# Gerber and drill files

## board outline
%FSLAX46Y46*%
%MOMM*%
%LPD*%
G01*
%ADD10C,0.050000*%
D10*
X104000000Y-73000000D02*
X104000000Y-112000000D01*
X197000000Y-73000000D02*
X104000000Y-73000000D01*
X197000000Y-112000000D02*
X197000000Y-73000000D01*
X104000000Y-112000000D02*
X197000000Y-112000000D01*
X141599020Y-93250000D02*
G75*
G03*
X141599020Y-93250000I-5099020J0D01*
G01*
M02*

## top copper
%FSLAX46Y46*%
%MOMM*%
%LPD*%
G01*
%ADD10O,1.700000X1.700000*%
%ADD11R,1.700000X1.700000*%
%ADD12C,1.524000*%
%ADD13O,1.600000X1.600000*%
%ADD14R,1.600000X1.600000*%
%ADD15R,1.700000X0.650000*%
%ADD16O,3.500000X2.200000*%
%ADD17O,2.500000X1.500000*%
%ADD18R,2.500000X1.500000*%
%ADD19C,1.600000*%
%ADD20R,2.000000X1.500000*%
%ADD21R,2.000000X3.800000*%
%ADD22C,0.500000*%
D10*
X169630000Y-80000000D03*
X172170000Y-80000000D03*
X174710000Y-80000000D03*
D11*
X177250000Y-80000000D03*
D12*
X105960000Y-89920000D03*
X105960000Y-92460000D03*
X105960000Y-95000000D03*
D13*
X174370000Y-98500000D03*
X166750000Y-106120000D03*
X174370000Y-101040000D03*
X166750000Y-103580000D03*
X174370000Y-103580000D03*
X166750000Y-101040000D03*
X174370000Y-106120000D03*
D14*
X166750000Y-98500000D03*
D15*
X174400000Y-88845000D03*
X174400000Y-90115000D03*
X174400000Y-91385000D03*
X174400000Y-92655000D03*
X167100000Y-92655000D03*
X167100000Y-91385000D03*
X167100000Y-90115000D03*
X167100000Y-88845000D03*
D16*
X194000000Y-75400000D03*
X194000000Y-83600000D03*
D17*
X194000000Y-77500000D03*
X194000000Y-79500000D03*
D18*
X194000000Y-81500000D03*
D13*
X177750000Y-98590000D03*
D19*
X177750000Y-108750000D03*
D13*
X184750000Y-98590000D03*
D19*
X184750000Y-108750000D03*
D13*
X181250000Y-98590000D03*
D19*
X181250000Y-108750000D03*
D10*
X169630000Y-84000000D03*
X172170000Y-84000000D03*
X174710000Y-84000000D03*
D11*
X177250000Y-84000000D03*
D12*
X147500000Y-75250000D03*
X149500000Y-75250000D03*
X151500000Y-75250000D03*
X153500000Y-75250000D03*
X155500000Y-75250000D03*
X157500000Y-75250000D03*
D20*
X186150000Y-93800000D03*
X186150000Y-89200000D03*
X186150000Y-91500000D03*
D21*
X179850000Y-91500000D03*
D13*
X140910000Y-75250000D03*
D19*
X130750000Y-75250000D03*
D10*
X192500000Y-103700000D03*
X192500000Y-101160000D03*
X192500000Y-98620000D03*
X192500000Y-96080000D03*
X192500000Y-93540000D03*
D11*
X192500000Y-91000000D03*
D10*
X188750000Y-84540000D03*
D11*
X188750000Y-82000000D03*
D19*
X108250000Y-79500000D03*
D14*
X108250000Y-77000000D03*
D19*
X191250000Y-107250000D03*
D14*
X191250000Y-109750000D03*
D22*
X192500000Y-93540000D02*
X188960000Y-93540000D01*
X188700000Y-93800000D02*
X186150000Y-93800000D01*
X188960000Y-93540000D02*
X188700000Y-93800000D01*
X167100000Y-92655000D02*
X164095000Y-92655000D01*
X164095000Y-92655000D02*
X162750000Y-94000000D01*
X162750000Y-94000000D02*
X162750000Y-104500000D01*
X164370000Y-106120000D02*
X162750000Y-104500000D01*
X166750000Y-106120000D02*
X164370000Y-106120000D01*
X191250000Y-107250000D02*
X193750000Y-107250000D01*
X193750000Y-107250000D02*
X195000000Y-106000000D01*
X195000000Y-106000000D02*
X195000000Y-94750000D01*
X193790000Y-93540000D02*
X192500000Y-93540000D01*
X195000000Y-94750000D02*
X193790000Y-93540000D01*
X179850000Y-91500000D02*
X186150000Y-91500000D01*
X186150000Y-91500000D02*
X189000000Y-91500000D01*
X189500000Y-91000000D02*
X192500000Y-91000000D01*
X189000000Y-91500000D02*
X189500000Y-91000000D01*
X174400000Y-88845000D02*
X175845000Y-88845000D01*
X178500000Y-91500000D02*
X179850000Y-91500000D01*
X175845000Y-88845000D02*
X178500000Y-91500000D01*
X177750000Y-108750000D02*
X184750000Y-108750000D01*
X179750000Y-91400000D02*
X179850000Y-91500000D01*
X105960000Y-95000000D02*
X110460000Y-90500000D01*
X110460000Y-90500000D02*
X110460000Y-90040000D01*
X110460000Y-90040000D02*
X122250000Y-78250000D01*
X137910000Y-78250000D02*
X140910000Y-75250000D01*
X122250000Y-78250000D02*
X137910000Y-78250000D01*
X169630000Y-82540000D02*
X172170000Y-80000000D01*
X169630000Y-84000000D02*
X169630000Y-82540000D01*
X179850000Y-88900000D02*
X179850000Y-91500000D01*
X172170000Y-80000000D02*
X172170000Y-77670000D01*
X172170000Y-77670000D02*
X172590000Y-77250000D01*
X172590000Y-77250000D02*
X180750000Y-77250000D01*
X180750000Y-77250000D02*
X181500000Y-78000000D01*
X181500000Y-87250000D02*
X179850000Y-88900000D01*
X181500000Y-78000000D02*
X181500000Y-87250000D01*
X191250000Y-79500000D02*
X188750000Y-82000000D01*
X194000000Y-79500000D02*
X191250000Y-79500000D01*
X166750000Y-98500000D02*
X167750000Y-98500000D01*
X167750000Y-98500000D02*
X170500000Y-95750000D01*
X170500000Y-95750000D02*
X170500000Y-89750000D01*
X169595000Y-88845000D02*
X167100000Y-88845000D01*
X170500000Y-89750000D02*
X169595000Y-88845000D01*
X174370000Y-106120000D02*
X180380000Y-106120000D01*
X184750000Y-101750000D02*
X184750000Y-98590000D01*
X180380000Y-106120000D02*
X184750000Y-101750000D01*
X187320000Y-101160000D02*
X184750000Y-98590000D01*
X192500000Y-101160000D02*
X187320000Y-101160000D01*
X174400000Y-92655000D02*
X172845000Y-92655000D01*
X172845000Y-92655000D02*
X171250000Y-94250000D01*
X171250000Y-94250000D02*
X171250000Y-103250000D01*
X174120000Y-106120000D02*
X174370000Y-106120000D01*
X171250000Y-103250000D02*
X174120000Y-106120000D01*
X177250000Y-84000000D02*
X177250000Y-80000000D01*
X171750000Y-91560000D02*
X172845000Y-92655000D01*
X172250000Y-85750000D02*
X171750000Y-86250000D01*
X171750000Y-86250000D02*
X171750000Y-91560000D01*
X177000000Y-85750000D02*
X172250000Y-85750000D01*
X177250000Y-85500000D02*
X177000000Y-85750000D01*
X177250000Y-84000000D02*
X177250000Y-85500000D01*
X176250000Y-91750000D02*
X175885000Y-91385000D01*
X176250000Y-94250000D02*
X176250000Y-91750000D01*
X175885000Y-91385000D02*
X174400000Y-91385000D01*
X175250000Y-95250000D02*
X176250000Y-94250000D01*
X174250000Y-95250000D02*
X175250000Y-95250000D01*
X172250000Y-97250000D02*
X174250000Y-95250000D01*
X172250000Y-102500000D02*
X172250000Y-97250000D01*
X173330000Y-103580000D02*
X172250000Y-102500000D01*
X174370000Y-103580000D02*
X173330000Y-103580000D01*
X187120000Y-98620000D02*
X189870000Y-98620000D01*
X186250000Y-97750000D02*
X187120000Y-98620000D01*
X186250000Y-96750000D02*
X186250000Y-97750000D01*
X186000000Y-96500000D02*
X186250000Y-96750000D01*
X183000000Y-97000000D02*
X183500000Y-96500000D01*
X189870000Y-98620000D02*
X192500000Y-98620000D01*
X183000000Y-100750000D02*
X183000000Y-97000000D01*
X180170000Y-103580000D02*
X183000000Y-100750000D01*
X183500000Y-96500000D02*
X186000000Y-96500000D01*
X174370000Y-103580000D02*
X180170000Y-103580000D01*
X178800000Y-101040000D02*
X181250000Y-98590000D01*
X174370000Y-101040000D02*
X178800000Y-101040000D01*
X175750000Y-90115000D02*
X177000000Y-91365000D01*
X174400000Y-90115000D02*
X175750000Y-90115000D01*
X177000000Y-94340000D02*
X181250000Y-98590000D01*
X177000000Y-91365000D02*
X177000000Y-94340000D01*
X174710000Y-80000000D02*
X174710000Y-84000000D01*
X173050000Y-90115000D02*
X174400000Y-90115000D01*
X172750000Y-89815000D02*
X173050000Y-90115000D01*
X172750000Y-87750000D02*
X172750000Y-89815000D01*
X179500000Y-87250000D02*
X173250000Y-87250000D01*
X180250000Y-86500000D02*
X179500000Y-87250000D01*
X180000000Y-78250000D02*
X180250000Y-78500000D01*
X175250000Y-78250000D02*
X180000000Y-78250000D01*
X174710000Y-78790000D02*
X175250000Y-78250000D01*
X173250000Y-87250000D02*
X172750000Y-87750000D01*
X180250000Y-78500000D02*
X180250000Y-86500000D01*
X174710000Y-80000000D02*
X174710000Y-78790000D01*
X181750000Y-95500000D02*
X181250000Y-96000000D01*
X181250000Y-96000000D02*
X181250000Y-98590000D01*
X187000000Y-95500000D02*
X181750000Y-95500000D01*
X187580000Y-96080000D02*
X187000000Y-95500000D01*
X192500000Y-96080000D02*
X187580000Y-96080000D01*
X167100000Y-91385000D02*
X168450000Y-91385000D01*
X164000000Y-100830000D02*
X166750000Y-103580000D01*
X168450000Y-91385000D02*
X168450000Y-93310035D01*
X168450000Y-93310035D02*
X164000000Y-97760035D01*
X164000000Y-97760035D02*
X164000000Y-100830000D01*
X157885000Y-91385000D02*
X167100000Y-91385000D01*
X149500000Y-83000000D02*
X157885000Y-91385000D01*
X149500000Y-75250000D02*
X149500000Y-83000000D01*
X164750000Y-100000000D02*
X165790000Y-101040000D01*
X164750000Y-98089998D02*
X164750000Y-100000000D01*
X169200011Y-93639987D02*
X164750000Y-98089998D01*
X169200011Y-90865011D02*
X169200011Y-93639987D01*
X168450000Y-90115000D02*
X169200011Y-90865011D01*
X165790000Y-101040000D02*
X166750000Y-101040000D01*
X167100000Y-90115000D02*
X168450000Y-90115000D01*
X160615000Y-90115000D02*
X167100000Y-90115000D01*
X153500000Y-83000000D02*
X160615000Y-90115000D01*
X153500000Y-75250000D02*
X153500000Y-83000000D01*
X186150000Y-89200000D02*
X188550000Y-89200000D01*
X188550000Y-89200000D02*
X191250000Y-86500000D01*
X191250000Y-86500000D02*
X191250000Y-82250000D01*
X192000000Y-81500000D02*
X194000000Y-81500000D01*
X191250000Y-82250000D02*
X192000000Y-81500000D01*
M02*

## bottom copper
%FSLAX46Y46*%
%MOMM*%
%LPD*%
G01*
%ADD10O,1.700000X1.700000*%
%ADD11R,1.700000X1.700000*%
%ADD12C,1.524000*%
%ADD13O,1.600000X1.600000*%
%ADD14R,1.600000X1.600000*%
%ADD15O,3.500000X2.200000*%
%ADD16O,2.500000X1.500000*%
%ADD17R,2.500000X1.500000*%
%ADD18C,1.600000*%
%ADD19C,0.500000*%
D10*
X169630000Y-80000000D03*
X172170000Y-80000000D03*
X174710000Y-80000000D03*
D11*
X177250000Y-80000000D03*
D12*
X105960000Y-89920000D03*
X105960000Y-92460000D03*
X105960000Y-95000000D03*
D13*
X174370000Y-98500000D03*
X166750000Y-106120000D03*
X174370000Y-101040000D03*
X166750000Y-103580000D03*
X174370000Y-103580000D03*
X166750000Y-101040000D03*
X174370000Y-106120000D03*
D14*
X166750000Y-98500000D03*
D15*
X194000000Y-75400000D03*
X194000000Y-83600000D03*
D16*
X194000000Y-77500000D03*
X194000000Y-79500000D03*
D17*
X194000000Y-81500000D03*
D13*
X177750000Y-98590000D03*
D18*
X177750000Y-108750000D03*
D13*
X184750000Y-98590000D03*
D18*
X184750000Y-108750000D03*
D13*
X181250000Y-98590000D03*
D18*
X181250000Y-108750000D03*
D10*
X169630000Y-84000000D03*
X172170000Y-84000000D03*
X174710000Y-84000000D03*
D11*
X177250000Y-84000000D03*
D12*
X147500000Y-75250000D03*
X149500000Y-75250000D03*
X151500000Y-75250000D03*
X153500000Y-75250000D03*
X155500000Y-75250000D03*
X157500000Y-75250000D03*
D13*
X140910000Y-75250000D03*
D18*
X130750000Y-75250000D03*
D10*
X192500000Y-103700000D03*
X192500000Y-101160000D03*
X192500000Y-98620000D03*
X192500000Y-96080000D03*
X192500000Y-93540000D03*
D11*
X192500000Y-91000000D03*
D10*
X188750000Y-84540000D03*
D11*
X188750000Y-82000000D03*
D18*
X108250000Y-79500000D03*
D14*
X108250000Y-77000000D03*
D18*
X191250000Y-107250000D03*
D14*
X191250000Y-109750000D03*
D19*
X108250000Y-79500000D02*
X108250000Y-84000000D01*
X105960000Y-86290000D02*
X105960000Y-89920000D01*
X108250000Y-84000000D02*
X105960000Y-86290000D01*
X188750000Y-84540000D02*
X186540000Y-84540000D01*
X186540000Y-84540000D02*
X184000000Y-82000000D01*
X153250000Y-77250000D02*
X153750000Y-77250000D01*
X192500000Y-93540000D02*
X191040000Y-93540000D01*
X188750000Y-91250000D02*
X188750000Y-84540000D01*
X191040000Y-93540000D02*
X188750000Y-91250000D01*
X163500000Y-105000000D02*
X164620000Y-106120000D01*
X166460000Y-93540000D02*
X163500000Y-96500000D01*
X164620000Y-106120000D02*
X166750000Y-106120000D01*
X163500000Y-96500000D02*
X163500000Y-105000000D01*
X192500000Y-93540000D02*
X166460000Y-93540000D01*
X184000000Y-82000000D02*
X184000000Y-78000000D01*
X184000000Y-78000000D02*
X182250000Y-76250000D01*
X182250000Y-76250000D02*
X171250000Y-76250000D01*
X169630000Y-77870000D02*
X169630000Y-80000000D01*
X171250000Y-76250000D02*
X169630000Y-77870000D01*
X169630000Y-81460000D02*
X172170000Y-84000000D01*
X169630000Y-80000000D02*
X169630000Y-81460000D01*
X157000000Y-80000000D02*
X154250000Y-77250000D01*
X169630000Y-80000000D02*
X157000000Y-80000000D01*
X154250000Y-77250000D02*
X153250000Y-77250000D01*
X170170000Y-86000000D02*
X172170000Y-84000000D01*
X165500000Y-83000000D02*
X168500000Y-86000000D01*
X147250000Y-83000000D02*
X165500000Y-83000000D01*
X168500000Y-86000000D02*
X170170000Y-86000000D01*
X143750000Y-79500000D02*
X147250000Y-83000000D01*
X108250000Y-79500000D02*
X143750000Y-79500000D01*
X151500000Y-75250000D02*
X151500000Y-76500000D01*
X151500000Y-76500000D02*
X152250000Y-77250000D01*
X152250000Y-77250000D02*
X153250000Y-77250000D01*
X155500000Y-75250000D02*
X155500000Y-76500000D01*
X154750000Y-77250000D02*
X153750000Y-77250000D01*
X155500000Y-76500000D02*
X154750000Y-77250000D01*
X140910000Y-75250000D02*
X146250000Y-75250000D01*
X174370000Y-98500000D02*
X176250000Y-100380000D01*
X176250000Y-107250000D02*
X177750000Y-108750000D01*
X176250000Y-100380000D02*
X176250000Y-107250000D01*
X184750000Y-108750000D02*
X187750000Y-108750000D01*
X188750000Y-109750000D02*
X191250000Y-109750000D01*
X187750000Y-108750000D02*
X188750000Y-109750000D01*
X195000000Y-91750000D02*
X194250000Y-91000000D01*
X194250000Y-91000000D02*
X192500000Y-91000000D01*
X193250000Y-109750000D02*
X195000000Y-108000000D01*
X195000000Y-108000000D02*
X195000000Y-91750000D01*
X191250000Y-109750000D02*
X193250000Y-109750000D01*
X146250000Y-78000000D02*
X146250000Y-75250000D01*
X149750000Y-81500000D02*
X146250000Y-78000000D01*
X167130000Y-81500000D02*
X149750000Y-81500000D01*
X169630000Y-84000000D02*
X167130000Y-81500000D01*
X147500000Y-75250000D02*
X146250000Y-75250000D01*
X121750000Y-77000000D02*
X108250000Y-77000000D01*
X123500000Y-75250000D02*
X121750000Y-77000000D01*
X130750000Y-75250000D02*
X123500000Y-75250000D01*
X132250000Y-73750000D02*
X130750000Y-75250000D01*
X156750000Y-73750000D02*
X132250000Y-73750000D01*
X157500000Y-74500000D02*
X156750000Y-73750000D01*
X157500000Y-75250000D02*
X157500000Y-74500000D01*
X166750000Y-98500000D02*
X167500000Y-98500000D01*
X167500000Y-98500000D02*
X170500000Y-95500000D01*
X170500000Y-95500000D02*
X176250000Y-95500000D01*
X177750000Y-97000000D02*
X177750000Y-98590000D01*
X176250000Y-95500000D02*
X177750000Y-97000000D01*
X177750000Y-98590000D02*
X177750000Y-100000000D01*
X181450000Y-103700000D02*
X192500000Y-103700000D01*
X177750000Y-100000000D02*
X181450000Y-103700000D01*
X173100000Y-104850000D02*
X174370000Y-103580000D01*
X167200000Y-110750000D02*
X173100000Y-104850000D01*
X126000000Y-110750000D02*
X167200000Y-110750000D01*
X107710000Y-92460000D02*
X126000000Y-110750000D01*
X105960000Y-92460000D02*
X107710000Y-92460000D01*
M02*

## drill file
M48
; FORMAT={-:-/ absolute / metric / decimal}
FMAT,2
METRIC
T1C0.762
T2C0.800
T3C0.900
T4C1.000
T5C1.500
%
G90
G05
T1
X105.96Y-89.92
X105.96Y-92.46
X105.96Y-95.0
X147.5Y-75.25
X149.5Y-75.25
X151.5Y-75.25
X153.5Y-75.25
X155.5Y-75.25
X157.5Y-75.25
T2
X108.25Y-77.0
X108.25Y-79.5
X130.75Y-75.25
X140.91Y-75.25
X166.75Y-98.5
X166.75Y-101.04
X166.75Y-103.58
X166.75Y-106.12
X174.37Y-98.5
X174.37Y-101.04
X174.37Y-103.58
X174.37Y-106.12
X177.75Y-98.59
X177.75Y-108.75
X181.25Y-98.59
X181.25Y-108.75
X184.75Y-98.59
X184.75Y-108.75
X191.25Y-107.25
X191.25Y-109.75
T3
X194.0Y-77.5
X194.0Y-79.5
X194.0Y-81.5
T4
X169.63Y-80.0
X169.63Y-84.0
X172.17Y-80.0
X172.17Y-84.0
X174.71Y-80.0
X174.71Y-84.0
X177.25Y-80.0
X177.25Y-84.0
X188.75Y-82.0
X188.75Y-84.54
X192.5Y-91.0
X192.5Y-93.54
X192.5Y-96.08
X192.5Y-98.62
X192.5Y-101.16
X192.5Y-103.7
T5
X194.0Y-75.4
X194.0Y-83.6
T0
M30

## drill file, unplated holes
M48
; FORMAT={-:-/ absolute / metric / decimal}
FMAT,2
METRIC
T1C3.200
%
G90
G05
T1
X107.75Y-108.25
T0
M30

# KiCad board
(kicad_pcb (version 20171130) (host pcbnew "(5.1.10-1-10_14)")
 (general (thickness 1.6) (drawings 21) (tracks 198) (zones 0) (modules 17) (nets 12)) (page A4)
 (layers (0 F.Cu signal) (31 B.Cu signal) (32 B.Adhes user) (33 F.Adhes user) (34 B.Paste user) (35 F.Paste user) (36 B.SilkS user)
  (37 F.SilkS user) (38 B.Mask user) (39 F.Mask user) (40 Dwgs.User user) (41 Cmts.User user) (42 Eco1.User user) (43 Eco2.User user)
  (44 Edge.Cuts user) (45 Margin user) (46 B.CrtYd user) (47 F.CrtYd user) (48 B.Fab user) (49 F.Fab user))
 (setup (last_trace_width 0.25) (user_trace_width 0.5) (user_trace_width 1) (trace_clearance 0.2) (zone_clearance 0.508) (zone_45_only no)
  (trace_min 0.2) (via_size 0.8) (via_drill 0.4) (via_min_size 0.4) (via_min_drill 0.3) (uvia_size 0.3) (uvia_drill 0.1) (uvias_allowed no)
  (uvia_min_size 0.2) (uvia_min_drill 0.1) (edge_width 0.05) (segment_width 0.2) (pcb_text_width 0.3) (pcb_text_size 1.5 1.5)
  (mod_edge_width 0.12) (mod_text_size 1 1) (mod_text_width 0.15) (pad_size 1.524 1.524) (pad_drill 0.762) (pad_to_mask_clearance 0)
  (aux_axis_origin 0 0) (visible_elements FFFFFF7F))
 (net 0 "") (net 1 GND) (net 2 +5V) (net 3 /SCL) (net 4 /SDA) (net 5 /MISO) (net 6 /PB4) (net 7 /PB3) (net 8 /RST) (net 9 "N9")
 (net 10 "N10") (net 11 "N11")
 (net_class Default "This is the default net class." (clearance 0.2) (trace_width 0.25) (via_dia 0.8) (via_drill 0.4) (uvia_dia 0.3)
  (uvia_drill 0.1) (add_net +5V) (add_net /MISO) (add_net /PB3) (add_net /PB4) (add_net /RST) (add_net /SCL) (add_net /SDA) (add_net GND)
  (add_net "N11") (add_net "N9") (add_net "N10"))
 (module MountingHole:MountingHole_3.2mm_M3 (layer F.Cu) (at 107.75 108.25)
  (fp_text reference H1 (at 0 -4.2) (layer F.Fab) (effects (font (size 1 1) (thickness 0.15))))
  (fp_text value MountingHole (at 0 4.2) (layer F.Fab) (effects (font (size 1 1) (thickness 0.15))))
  (pad 1 np_thru_hole circle (at 0 0) (size 3.2 3.2) (drill 3.2) (layers *.Cu *.Mask)))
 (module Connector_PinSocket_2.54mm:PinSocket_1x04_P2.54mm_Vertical (layer F.Cu) (at 177.25 80 270)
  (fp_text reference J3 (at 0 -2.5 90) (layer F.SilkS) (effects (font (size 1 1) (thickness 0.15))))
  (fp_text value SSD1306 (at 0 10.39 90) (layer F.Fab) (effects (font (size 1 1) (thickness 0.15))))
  (pad 4 thru_hole oval (at 0 7.62 270) (size 1.7 1.7) (drill 1) (layers *.Cu *.Mask) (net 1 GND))
  (pad 3 thru_hole oval (at 0 5.08 270) (size 1.7 1.7) (drill 1) (layers *.Cu *.Mask) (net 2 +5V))
  (pad 2 thru_hole oval (at 0 2.54 270) (size 1.7 1.7) (drill 1) (layers *.Cu *.Mask) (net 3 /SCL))
  (pad 1 thru_hole rect (at 0 0 270) (size 1.7 1.7) (drill 1) (layers *.Cu *.Mask) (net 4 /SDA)))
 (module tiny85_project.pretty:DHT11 (layer F.Cu) (at 104.5 86 270)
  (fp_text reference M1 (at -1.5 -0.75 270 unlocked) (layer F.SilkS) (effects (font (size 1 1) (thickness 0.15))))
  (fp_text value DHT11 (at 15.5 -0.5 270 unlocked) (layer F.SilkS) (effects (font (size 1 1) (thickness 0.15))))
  (pad 3 thru_hole circle (at 3.92 -1.46 90) (size 1.524 1.524) (drill 0.762) (layers *.Cu *.Mask) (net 1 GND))
  (pad 2 thru_hole circle (at 6.46 -1.46 90) (size 1.524 1.524) (drill 0.762) (layers *.Cu *.Mask) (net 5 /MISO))
  (pad 1 thru_hole circle (at 9 -1.46 90) (size 1.524 1.524) (drill 0.762) (layers *.Cu *.Mask) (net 2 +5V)))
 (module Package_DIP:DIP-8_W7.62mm (layer F.Cu) (at 166.75 98.5)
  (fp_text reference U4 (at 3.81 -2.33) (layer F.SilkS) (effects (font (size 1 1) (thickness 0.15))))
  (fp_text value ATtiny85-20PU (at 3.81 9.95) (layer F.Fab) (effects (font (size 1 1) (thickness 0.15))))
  (pad 8 thru_hole oval (at 7.62 0) (size 1.6 1.6) (drill 0.8) (layers *.Cu *.Mask) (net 2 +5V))
  (pad 4 thru_hole oval (at 0 7.62) (size 1.6 1.6) (drill 0.8) (layers *.Cu *.Mask) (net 1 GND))
  (pad 7 thru_hole oval (at 7.62 2.54) (size 1.6 1.6) (drill 0.8) (layers *.Cu *.Mask) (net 3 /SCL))
  (pad 3 thru_hole oval (at 0 5.08) (size 1.6 1.6) (drill 0.8) (layers *.Cu *.Mask) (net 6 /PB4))
  (pad 6 thru_hole oval (at 7.62 5.08) (size 1.6 1.6) (drill 0.8) (layers *.Cu *.Mask) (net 5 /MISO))
  (pad 2 thru_hole oval (at 0 2.54) (size 1.6 1.6) (drill 0.8) (layers *.Cu *.Mask) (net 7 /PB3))
  (pad 5 thru_hole oval (at 7.62 7.62) (size 1.6 1.6) (drill 0.8) (layers *.Cu *.Mask) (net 4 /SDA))
  (pad 1 thru_hole rect (at 0 0) (size 1.6 1.6) (drill 0.8) (layers *.Cu *.Mask) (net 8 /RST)))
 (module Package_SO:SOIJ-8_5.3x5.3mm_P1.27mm (layer F.Cu) (at 170.75 90.75)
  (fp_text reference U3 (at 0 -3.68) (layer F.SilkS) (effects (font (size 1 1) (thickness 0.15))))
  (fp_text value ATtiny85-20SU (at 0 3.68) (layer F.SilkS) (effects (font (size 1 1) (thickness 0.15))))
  (pad 8 smd rect (at 3.65 -1.905) (size 1.7 0.65) (layers F.Cu F.Paste F.Mask) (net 2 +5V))
  (pad 7 smd rect (at 3.65 -0.635) (size 1.7 0.65) (layers F.Cu F.Paste F.Mask) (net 3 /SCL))
  (pad 6 smd rect (at 3.65 0.635) (size 1.7 0.65) (layers F.Cu F.Paste F.Mask) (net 5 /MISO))
  (pad 5 smd rect (at 3.65 1.905) (size 1.7 0.65) (layers F.Cu F.Paste F.Mask) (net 4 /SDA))
  (pad 4 smd rect (at -3.65 1.905) (size 1.7 0.65) (layers F.Cu F.Paste F.Mask) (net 1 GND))
  (pad 3 smd rect (at -3.65 0.635) (size 1.7 0.65) (layers F.Cu F.Paste F.Mask) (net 6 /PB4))
  (pad 2 smd rect (at -3.65 -0.635) (size 1.7 0.65) (layers F.Cu F.Paste F.Mask) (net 7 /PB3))
  (pad 1 smd rect (at -3.65 -1.905) (size 1.7 0.65) (layers F.Cu F.Paste F.Mask) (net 8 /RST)))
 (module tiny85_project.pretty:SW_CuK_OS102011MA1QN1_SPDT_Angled (layer F.Cu) (at 194 81.5 90)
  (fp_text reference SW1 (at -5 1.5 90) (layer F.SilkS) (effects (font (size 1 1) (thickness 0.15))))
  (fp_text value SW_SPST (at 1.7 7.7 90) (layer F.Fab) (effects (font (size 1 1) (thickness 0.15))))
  (pad "" thru_hole oval (at 6.1 0 90) (size 2.2 3.5) (drill 1.5) (layers *.Cu *.Mask))
  (pad "" thru_hole oval (at -2.1 0 90) (size 2.2 3.5) (drill 1.5) (layers *.Cu *.Mask))
  (pad 3 thru_hole oval (at 4 0 90) (size 1.5 2.5) (drill 0.9) (layers *.Cu *.Mask))
  (pad 2 thru_hole oval (at 2 0 90) (size 1.5 2.5) (drill 0.9) (layers *.Cu *.Mask) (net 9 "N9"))
  (pad 1 thru_hole rect (at 0 0 90) (size 1.5 2.5) (drill 0.9) (layers *.Cu *.Mask) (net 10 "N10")))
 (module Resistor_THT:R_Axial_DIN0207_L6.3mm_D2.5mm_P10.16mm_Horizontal (layer F.Cu) (at 177.75 108.75 90)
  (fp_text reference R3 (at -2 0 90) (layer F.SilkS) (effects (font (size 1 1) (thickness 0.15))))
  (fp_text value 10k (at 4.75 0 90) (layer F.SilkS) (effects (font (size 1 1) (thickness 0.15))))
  (pad 2 thru_hole oval (at 10.16 0 90) (size 1.6 1.6) (drill 0.8) (layers *.Cu *.Mask) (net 8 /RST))
  (pad 1 thru_hole circle (at 0 0 90) (size 1.6 1.6) (drill 0.8) (layers *.Cu *.Mask) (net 2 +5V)))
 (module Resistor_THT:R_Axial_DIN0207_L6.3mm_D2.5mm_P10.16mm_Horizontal (layer F.Cu) (at 184.75 108.75 90)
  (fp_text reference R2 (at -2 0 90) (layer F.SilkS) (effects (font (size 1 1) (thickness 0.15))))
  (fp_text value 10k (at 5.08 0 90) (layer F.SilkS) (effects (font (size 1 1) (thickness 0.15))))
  (pad 2 thru_hole oval (at 10.16 0 90) (size 1.6 1.6) (drill 0.8) (layers *.Cu *.Mask) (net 4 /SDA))
  (pad 1 thru_hole circle (at 0 0 90) (size 1.6 1.6) (drill 0.8) (layers *.Cu *.Mask) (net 2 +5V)))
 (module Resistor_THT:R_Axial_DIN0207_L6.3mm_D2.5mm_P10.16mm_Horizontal (layer F.Cu) (at 181.25 108.75 90)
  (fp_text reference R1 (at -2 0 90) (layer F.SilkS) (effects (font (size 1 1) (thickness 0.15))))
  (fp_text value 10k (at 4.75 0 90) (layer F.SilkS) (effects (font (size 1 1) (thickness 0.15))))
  (pad 2 thru_hole oval (at 10.16 0 90) (size 1.6 1.6) (drill 0.8) (layers *.Cu *.Mask) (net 3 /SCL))
  (pad 1 thru_hole circle (at 0 0 90) (size 1.6 1.6) (drill 0.8) (layers *.Cu *.Mask) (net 2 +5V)))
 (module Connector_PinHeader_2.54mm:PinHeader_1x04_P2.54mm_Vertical (layer F.Cu) (at 177.25 84 270)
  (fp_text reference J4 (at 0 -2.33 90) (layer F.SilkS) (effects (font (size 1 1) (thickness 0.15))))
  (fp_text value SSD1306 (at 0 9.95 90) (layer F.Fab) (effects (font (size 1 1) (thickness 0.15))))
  (pad 4 thru_hole oval (at 0 7.62 270) (size 1.7 1.7) (drill 1) (layers *.Cu *.Mask) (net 2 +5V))
  (pad 3 thru_hole oval (at 0 5.08 270) (size 1.7 1.7) (drill 1) (layers *.Cu *.Mask) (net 1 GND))
  (pad 2 thru_hole oval (at 0 2.54 270) (size 1.7 1.7) (drill 1) (layers *.Cu *.Mask) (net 3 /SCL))
  (pad 1 thru_hole rect (at 0 0 270) (size 1.7 1.7) (drill 1) (layers *.Cu *.Mask) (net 4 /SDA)))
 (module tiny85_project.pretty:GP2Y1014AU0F (layer F.Cu) (at 159.5 77.25 180)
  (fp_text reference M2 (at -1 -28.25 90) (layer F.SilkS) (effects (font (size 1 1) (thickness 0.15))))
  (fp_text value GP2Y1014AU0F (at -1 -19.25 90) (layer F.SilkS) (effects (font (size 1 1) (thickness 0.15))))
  (pad 6 thru_hole circle (at 12 2 180) (size 1.524 1.524) (drill 0.762) (layers *.Cu *.Mask) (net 2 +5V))
  (pad 5 thru_hole circle (at 10 2 180) (size 1.524 1.524) (drill 0.762) (layers *.Cu *.Mask) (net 6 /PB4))
  (pad 4 thru_hole circle (at 8 2 180) (size 1.524 1.524) (drill 0.762) (layers *.Cu *.Mask) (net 1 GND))
  (pad 3 thru_hole circle (at 6 2 180) (size 1.524 1.524) (drill 0.762) (layers *.Cu *.Mask) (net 7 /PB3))
  (pad 2 thru_hole circle (at 4 2 180) (size 1.524 1.524) (drill 0.762) (layers *.Cu *.Mask) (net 1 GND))
  (pad 1 thru_hole circle (at 2 2 180) (size 1.524 1.524) (drill 0.762) (layers *.Cu *.Mask) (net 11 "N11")))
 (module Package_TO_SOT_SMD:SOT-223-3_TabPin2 (layer F.Cu) (at 183 91.5 180)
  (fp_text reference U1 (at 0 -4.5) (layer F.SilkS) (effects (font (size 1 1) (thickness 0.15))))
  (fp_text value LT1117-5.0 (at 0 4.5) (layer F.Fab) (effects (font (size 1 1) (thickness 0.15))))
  (pad 1 smd rect (at -3.15 -2.3 180) (size 2 1.5) (layers F.Cu F.Paste F.Mask) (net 1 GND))
  (pad 3 smd rect (at -3.15 2.3 180) (size 2 1.5) (layers F.Cu F.Paste F.Mask) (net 10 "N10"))
  (pad 2 smd rect (at -3.15 0 180) (size 2 1.5) (layers F.Cu F.Paste F.Mask) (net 2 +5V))
  (pad 2 smd rect (at 3.15 0 180) (size 2 3.8) (layers F.Cu F.Paste F.Mask) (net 2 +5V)))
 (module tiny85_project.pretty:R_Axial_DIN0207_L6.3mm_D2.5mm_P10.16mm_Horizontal (layer F.Cu) (at 130.75 75.25)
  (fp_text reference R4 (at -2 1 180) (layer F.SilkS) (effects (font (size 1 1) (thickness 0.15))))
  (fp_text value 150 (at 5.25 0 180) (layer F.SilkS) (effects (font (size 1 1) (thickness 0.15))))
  (pad 2 thru_hole oval (at 10.16 0) (size 1.6 1.6) (drill 0.8) (layers *.Cu *.Mask) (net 2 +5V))
  (pad 1 thru_hole circle (at 0 0) (size 1.6 1.6) (drill 0.8) (layers *.Cu *.Mask) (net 11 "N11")))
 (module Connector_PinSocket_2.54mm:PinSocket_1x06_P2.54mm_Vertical (layer F.Cu) (at 192.5 91)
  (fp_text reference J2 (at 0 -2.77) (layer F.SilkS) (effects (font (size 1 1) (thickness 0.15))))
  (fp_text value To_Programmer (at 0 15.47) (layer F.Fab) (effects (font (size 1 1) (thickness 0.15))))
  (pad 6 thru_hole oval (at 0 12.7) (size 1.7 1.7) (drill 1) (layers *.Cu *.Mask) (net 8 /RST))
  (pad 5 thru_hole oval (at 0 10.16) (size 1.7 1.7) (drill 1) (layers *.Cu *.Mask) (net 4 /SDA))
  (pad 4 thru_hole oval (at 0 7.62) (size 1.7 1.7) (drill 1) (layers *.Cu *.Mask) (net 5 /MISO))
  (pad 3 thru_hole oval (at 0 5.08) (size 1.7 1.7) (drill 1) (layers *.Cu *.Mask) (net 3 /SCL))
  (pad 2 thru_hole oval (at 0 2.54) (size 1.7 1.7) (drill 1) (layers *.Cu *.Mask) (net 1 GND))
  (pad 1 thru_hole rect (at 0 0) (size 1.7 1.7) (drill 1) (layers *.Cu *.Mask) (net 2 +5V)))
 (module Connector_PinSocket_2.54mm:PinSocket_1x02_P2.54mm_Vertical (layer F.Cu) (at 188.75 82)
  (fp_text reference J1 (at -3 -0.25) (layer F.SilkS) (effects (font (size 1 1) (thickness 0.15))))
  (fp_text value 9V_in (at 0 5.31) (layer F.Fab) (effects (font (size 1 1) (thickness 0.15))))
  (pad 2 thru_hole oval (at 0 2.54) (size 1.7 1.7) (drill 1) (layers *.Cu *.Mask) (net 1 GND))
  (pad 1 thru_hole rect (at 0 0) (size 1.7 1.7) (drill 1) (layers *.Cu *.Mask) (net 9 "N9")))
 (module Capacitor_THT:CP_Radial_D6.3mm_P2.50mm (layer F.Cu) (at 108.25 77 270)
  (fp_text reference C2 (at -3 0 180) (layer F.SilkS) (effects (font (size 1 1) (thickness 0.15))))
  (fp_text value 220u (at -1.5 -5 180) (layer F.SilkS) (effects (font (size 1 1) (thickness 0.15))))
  (pad 2 thru_hole circle (at 2.5 0 270) (size 1.6 1.6) (drill 0.8) (layers *.Cu *.Mask) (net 1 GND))
  (pad 1 thru_hole rect (at 0 0 270) (size 1.6 1.6) (drill 0.8) (layers *.Cu *.Mask) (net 11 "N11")))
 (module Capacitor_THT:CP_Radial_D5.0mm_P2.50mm (layer F.Cu) (at 191.25 109.75 90)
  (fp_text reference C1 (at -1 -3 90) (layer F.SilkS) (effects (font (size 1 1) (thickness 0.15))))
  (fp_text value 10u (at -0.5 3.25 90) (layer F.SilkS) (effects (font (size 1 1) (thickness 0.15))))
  (pad 2 thru_hole circle (at 2.5 0 90) (size 1.6 1.6) (drill 0.8) (layers *.Cu *.Mask) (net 1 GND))
  (pad 1 thru_hole rect (at 0 0 90) (size 1.6 1.6) (drill 0.8) (layers *.Cu *.Mask) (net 2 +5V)))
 (gr_line (start 104 73) (end 104 112) (layer Edge.Cuts) (width 0.05))
 (gr_line (start 197 73) (end 104 73) (layer Edge.Cuts) (width 0.05))
 (gr_line (start 197 112) (end 197 73) (layer Edge.Cuts) (width 0.05))
 (gr_line (start 104 112) (end 197 112) (layer Edge.Cuts) (width 0.05))
 (gr_circle (center 136.5 93.25) (end 141.5 94.25) (layer Edge.Cuts) (width 0.05))
 (segment (start 108.25 79.5) (end 108.25 84) (width 0.5) (layer B.Cu) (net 1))
 (segment (start 105.96 86.29) (end 105.96 89.92) (width 0.5) (layer B.Cu) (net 1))
 (segment (start 108.25 84) (end 105.96 86.29) (width 0.5) (layer B.Cu) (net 1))
 (segment (start 192.5 93.54) (end 188.96 93.54) (width 0.5) (layer F.Cu) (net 1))
 (segment (start 188.7 93.8) (end 186.15 93.8) (width 0.5) (layer F.Cu) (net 1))
 (segment (start 188.96 93.54) (end 188.7 93.8) (width 0.5) (layer F.Cu) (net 1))
 (segment (start 167.1 92.655) (end 164.095 92.655) (width 0.5) (layer F.Cu) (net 1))
 (segment (start 164.095 92.655) (end 162.75 94) (width 0.5) (layer F.Cu) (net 1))
 (segment (start 162.75 94) (end 162.75 104.5) (width 0.5) (layer F.Cu) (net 1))
 (segment (start 188.75 84.54) (end 186.54 84.54) (width 0.5) (layer B.Cu) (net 1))
 (segment (start 186.54 84.54) (end 184 82) (width 0.5) (layer B.Cu) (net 1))
 (segment (start 153.25 77.25) (end 153.75 77.25) (width 0.5) (layer B.Cu) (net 1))
 (segment (start 192.5 93.54) (end 191.04 93.54) (width 0.5) (layer B.Cu) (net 1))
 (segment (start 188.75 91.25) (end 188.75 84.54) (width 0.5) (layer B.Cu) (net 1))
 (segment (start 191.04 93.54) (end 188.75 91.25) (width 0.5) (layer B.Cu) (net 1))
 (segment (start 163.5 105) (end 164.62 106.12) (width 0.5) (layer B.Cu) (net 1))
 (segment (start 166.46 93.54) (end 163.5 96.5) (width 0.5) (layer B.Cu) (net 1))
 (segment (start 164.62 106.12) (end 166.75 106.12) (width 0.5) (layer B.Cu) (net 1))
 (segment (start 163.5 96.5) (end 163.5 105) (width 0.5) (layer B.Cu) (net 1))
 (segment (start 192.5 93.54) (end 166.46 93.54) (width 0.5) (layer B.Cu) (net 1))
 (segment (start 164.37 106.12) (end 162.75 104.5) (width 0.5) (layer F.Cu) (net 1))
 (segment (start 166.75 106.12) (end 164.37 106.12) (width 0.5) (layer F.Cu) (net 1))
 (segment (start 191.25 107.25) (end 193.75 107.25) (width 0.5) (layer F.Cu) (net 1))
 (segment (start 193.75 107.25) (end 195 106) (width 0.5) (layer F.Cu) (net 1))
 (segment (start 195 106) (end 195 94.75) (width 0.5) (layer F.Cu) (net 1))
 (segment (start 193.79 93.54) (end 192.5 93.54) (width 0.5) (layer F.Cu) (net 1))
 (segment (start 195 94.75) (end 193.79 93.54) (width 0.5) (layer F.Cu) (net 1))
 (segment (start 184 82) (end 184 78) (width 0.5) (layer B.Cu) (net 1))
 (segment (start 184 78) (end 182.25 76.25) (width 0.5) (layer B.Cu) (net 1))
 (segment (start 182.25 76.25) (end 171.25 76.25) (width 0.5) (layer B.Cu) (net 1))
 (segment (start 169.63 77.87) (end 169.63 80) (width 0.5) (layer B.Cu) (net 1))
 (segment (start 171.25 76.25) (end 169.63 77.87) (width 0.5) (layer B.Cu) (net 1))
 (segment (start 169.63 81.46) (end 172.17 84) (width 0.5) (layer B.Cu) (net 1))
 (segment (start 169.63 80) (end 169.63 81.46) (width 0.5) (layer B.Cu) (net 1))
 (segment (start 157 80) (end 154.25 77.25) (width 0.5) (layer B.Cu) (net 1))
 (segment (start 169.63 80) (end 157 80) (width 0.5) (layer B.Cu) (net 1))
 (segment (start 154.25 77.25) (end 153.25 77.25) (width 0.5) (layer B.Cu) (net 1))
 (segment (start 170.17 86) (end 172.17 84) (width 0.5) (layer B.Cu) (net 1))
 (segment (start 165.5 83) (end 168.5 86) (width 0.5) (layer B.Cu) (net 1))
 (segment (start 147.25 83) (end 165.5 83) (width 0.5) (layer B.Cu) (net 1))
 (segment (start 168.5 86) (end 170.17 86) (width 0.5) (layer B.Cu) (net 1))
 (segment (start 143.75 79.5) (end 147.25 83) (width 0.5) (layer B.Cu) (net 1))
 (segment (start 108.25 79.5) (end 143.75 79.5) (width 0.5) (layer B.Cu) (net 1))
 (segment (start 151.5 75.25) (end 151.5 76.5) (width 0.5) (layer B.Cu) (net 1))
 (segment (start 151.5 76.5) (end 152.25 77.25) (width 0.5) (layer B.Cu) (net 1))
 (segment (start 152.25 77.25) (end 153.25 77.25) (width 0.5) (layer B.Cu) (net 1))
 (segment (start 155.5 75.25) (end 155.5 76.5) (width 0.5) (layer B.Cu) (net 1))
 (segment (start 154.75 77.25) (end 153.75 77.25) (width 0.5) (layer B.Cu) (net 1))
 (segment (start 155.5 76.5) (end 154.75 77.25) (width 0.5) (layer B.Cu) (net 1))
 (segment (start 179.85 91.5) (end 186.15 91.5) (width 0.5) (layer F.Cu) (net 2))
 (segment (start 186.15 91.5) (end 189 91.5) (width 0.5) (layer F.Cu) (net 2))
 (segment (start 189.5 91) (end 192.5 91) (width 0.5) (layer F.Cu) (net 2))
 (segment (start 189 91.5) (end 189.5 91) (width 0.5) (layer F.Cu) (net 2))
 (segment (start 174.4 88.845) (end 175.845 88.845) (width 0.5) (layer F.Cu) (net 2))
 (segment (start 178.5 91.5) (end 179.85 91.5) (width 0.5) (layer F.Cu) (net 2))
 (segment (start 175.845 88.845) (end 178.5 91.5) (width 0.5) (layer F.Cu) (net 2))
 (segment (start 177.75 108.75) (end 184.75 108.75) (width 0.5) (layer F.Cu) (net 2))
 (segment (start 140.91 75.25) (end 146.25 75.25) (width 0.5) (layer B.Cu) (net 2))
 (segment (start 179.75 91.4) (end 179.85 91.5) (width 0.5) (layer F.Cu) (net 2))
 (segment (start 174.37 98.5) (end 176.25 100.38) (width 0.5) (layer B.Cu) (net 2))
 (segment (start 176.25 107.25) (end 177.75 108.75) (width 0.5) (layer B.Cu) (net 2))
 (segment (start 176.25 100.38) (end 176.25 107.25) (width 0.5) (layer B.Cu) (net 2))
 (segment (start 105.96 95) (end 110.46 90.5) (width 0.5) (layer F.Cu) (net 2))
 (segment (start 110.46 90.5) (end 110.46 90.04) (width 0.5) (layer F.Cu) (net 2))
 (segment (start 110.46 90.04) (end 122.25 78.25) (width 0.5) (layer F.Cu) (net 2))
 (segment (start 137.91 78.25) (end 140.91 75.25) (width 0.5) (layer F.Cu) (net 2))
 (segment (start 122.25 78.25) (end 137.91 78.25) (width 0.5) (layer F.Cu) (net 2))
 (segment (start 184.75 108.75) (end 187.75 108.75) (width 0.5) (layer B.Cu) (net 2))
 (segment (start 188.75 109.75) (end 191.25 109.75) (width 0.5) (layer B.Cu) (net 2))
 (segment (start 187.75 108.75) (end 188.75 109.75) (width 0.5) (layer B.Cu) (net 2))
 (segment (start 195 91.75) (end 194.25 91) (width 0.5) (layer B.Cu) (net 2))
 (segment (start 194.25 91) (end 192.5 91) (width 0.5) (layer B.Cu) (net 2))
 (segment (start 193.25 109.75) (end 195 108) (width 0.5) (layer B.Cu) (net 2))
 (segment (start 195 108) (end 195 91.75) (width 0.5) (layer B.Cu) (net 2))
 (segment (start 191.25 109.75) (end 193.25 109.75) (width 0.5) (layer B.Cu) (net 2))
 (segment (start 169.63 82.54) (end 172.17 80) (width 0.5) (layer F.Cu) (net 2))
 (segment (start 169.63 84) (end 169.63 82.54) (width 0.5) (layer F.Cu) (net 2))
 (segment (start 179.85 88.9) (end 179.85 91.5) (width 0.5) (layer F.Cu) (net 2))
 (segment (start 146.25 78) (end 146.25 75.25) (width 0.5) (layer B.Cu) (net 2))
 (segment (start 149.75 81.5) (end 146.25 78) (width 0.5) (layer B.Cu) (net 2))
 (segment (start 167.13 81.5) (end 149.75 81.5) (width 0.5) (layer B.Cu) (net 2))
 (segment (start 169.63 84) (end 167.13 81.5) (width 0.5) (layer B.Cu) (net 2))
 (segment (start 172.17 80) (end 172.17 77.67) (width 0.5) (layer F.Cu) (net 2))
 (segment (start 172.17 77.67) (end 172.59 77.25) (width 0.5) (layer F.Cu) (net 2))
 (segment (start 172.59 77.25) (end 180.75 77.25) (width 0.5) (layer F.Cu) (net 2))
 (segment (start 180.75 77.25) (end 181.5 78) (width 0.5) (layer F.Cu) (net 2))
 (segment (start 181.5 87.25) (end 179.85 88.9) (width 0.5) (layer F.Cu) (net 2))
 (segment (start 181.5 78) (end 181.5 87.25) (width 0.5) (layer F.Cu) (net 2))
 (segment (start 147.5 75.25) (end 146.25 75.25) (width 0.5) (layer B.Cu) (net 2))
 (segment (start 121.75 77) (end 108.25 77) (width 0.5) (layer B.Cu) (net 11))
 (segment (start 123.5 75.25) (end 121.75 77) (width 0.5) (layer B.Cu) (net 11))
 (segment (start 130.75 75.25) (end 123.5 75.25) (width 0.5) (layer B.Cu) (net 11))
 (segment (start 132.25 73.75) (end 130.75 75.25) (width 0.5) (layer B.Cu) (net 11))
 (segment (start 156.75 73.75) (end 132.25 73.75) (width 0.5) (layer B.Cu) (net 11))
 (segment (start 157.5 74.5) (end 156.75 73.75) (width 0.5) (layer B.Cu) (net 11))
 (segment (start 157.5 75.25) (end 157.5 74.5) (width 0.5) (layer B.Cu) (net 11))
 (segment (start 191.25 79.5) (end 188.75 82) (width 0.5) (layer F.Cu) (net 9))
 (segment (start 194 79.5) (end 191.25 79.5) (width 0.5) (layer F.Cu) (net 9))
 (segment (start 166.75 98.5) (end 167.75 98.5) (width 0.5) (layer F.Cu) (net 8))
 (segment (start 167.75 98.5) (end 170.5 95.75) (width 0.5) (layer F.Cu) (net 8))
 (segment (start 170.5 95.75) (end 170.5 89.75) (width 0.5) (layer F.Cu) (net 8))
 (segment (start 169.595 88.845) (end 167.1 88.845) (width 0.5) (layer F.Cu) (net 8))
 (segment (start 170.5 89.75) (end 169.595 88.845) (width 0.5) (layer F.Cu) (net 8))
 (segment (start 166.75 98.5) (end 167.5 98.5) (width 0.5) (layer B.Cu) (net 8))
 (segment (start 167.5 98.5) (end 170.5 95.5) (width 0.5) (layer B.Cu) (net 8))
 (segment (start 170.5 95.5) (end 176.25 95.5) (width 0.5) (layer B.Cu) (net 8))
 (segment (start 177.75 97) (end 177.75 98.59) (width 0.5) (layer B.Cu) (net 8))
 (segment (start 176.25 95.5) (end 177.75 97) (width 0.5) (layer B.Cu) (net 8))
 (segment (start 177.75 98.59) (end 177.75 100) (width 0.5) (layer B.Cu) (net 8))
 (segment (start 181.45 103.7) (end 192.5 103.7) (width 0.5) (layer B.Cu) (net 8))
 (segment (start 177.75 100) (end 181.45 103.7) (width 0.5) (layer B.Cu) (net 8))
 (segment (start 174.37 106.12) (end 180.38 106.12) (width 0.5) (layer F.Cu) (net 4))
 (segment (start 184.75 101.75) (end 184.75 98.59) (width 0.5) (layer F.Cu) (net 4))
 (segment (start 180.38 106.12) (end 184.75 101.75) (width 0.5) (layer F.Cu) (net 4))
 (segment (start 187.32 101.16) (end 184.75 98.59) (width 0.5) (layer F.Cu) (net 4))
 (segment (start 192.5 101.16) (end 187.32 101.16) (width 0.5) (layer F.Cu) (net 4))
 (segment (start 174.4 92.655) (end 172.845 92.655) (width 0.5) (layer F.Cu) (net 4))
 (segment (start 172.845 92.655) (end 171.25 94.25) (width 0.5) (layer F.Cu) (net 4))
 (segment (start 171.25 94.25) (end 171.25 103.25) (width 0.5) (layer F.Cu) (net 4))
 (segment (start 174.12 106.12) (end 174.37 106.12) (width 0.5) (layer F.Cu) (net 4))
 (segment (start 171.25 103.25) (end 174.12 106.12) (width 0.5) (layer F.Cu) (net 4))
 (segment (start 177.25 84) (end 177.25 80) (width 0.5) (layer F.Cu) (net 4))
 (segment (start 171.75 91.56) (end 172.845 92.655) (width 0.5) (layer F.Cu) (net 4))
 (segment (start 172.25 85.75) (end 171.75 86.25) (width 0.5) (layer F.Cu) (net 4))
 (segment (start 171.75 86.25) (end 171.75 91.56) (width 0.5) (layer F.Cu) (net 4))
 (segment (start 177 85.75) (end 172.25 85.75) (width 0.5) (layer F.Cu) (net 4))
 (segment (start 177.25 85.5) (end 177 85.75) (width 0.5) (layer F.Cu) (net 4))
 (segment (start 177.25 84) (end 177.25 85.5) (width 0.5) (layer F.Cu) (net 4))
 (segment (start 176.25 91.75) (end 175.885 91.385) (width 0.5) (layer F.Cu) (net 5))
 (segment (start 176.25 94.25) (end 176.25 91.75) (width 0.5) (layer F.Cu) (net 5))
 (segment (start 175.885 91.385) (end 174.4 91.385) (width 0.5) (layer F.Cu) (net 5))
 (segment (start 175.25 95.25) (end 176.25 94.25) (width 0.5) (layer F.Cu) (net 5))
 (segment (start 174.25 95.25) (end 175.25 95.25) (width 0.5) (layer F.Cu) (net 5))
 (segment (start 172.25 97.25) (end 174.25 95.25) (width 0.5) (layer F.Cu) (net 5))
 (segment (start 172.25 102.5) (end 172.25 97.25) (width 0.5) (layer F.Cu) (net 5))
 (segment (start 173.33 103.58) (end 172.25 102.5) (width 0.5) (layer F.Cu) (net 5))
 (segment (start 174.37 103.58) (end 173.33 103.58) (width 0.5) (layer F.Cu) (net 5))
 (segment (start 173.1 104.85) (end 174.37 103.58) (width 0.5) (layer B.Cu) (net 5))
 (segment (start 167.2 110.75) (end 173.1 104.85) (width 0.5) (layer B.Cu) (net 5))
 (segment (start 126 110.75) (end 167.2 110.75) (width 0.5) (layer B.Cu) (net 5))
 (segment (start 107.71 92.46) (end 126 110.75) (width 0.5) (layer B.Cu) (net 5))
 (segment (start 105.96 92.46) (end 107.71 92.46) (width 0.5) (layer B.Cu) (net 5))
 (segment (start 187.12 98.62) (end 189.87 98.62) (width 0.5) (layer F.Cu) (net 5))
 (segment (start 186.25 97.75) (end 187.12 98.62) (width 0.5) (layer F.Cu) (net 5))
 (segment (start 186.25 96.75) (end 186.25 97.75) (width 0.5) (layer F.Cu) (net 5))
 (segment (start 186 96.5) (end 186.25 96.75) (width 0.5) (layer F.Cu) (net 5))
 (segment (start 183 97) (end 183.5 96.5) (width 0.5) (layer F.Cu) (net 5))
 (segment (start 189.87 98.62) (end 192.5 98.62) (width 0.5) (layer F.Cu) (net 5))
 (segment (start 183 100.75) (end 183 97) (width 0.5) (layer F.Cu) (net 5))
 (segment (start 180.17 103.58) (end 183 100.75) (width 0.5) (layer F.Cu) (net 5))
 (segment (start 183.5 96.5) (end 186 96.5) (width 0.5) (layer F.Cu) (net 5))
 (segment (start 174.37 103.58) (end 180.17 103.58) (width 0.5) (layer F.Cu) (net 5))
 (segment (start 178.8 101.04) (end 181.25 98.59) (width 0.5) (layer F.Cu) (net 3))
 (segment (start 174.37 101.04) (end 178.8 101.04) (width 0.5) (layer F.Cu) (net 3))
 (segment (start 175.75 90.115) (end 177 91.365) (width 0.5) (layer F.Cu) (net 3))
 (segment (start 174.4 90.115) (end 175.75 90.115) (width 0.5) (layer F.Cu) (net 3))
 (segment (start 177 94.34) (end 181.25 98.59) (width 0.5) (layer F.Cu) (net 3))
 (segment (start 177 91.365) (end 177 94.34) (width 0.5) (layer F.Cu) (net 3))
 (segment (start 174.71 80) (end 174.71 84) (width 0.5) (layer F.Cu) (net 3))
 (segment (start 173.05 90.115) (end 174.4 90.115) (width 0.5) (layer F.Cu) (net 3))
 (segment (start 172.75 89.815) (end 173.05 90.115) (width 0.5) (layer F.Cu) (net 3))
 (segment (start 172.75 87.75) (end 172.75 89.815) (width 0.5) (layer F.Cu) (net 3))
 (segment (start 179.5 87.25) (end 173.25 87.25) (width 0.5) (layer F.Cu) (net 3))
 (segment (start 180.25 86.5) (end 179.5 87.25) (width 0.5) (layer F.Cu) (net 3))
 (segment (start 180 78.25) (end 180.25 78.5) (width 0.5) (layer F.Cu) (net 3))
 (segment (start 175.25 78.25) (end 180 78.25) (width 0.5) (layer F.Cu) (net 3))
 (segment (start 174.71 78.79) (end 175.25 78.25) (width 0.5) (layer F.Cu) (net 3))
 (segment (start 173.25 87.25) (end 172.75 87.75) (width 0.5) (layer F.Cu) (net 3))
 (segment (start 180.25 78.5) (end 180.25 86.5) (width 0.5) (layer F.Cu) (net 3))
 (segment (start 174.71 80) (end 174.71 78.79) (width 0.5) (layer F.Cu) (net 3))
 (segment (start 181.75 95.5) (end 181.25 96) (width 0.5) (layer F.Cu) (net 3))
 (segment (start 181.25 96) (end 181.25 98.59) (width 0.5) (layer F.Cu) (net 3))
 (segment (start 187 95.5) (end 181.75 95.5) (width 0.5) (layer F.Cu) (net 3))
 (segment (start 187.58 96.08) (end 187 95.5) (width 0.5) (layer F.Cu) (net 3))
 (segment (start 192.5 96.08) (end 187.58 96.08) (width 0.5) (layer F.Cu) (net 3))
 (segment (start 167.1 91.385) (end 168.45 91.385) (width 0.5) (layer F.Cu) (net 6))
 (segment (start 164 100.83) (end 166.75 103.58) (width 0.5) (layer F.Cu) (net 6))
 (segment (start 168.45 91.385) (end 168.45 93.310035) (width 0.5) (layer F.Cu) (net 6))
 (segment (start 168.45 93.310035) (end 164 97.760035) (width 0.5) (layer F.Cu) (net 6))
 (segment (start 164 97.760035) (end 164 100.83) (width 0.5) (layer F.Cu) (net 6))
 (segment (start 157.885 91.385) (end 167.1 91.385) (width 0.5) (layer F.Cu) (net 6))
 (segment (start 149.5 83) (end 157.885 91.385) (width 0.5) (layer F.Cu) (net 6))
 (segment (start 149.5 75.25) (end 149.5 83) (width 0.5) (layer F.Cu) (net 6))
 (segment (start 164.75 100) (end 165.79 101.04) (width 0.5) (layer F.Cu) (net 7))
 (segment (start 164.75 98.089998) (end 164.75 100) (width 0.5) (layer F.Cu) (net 7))
 (segment (start 169.200011 93.639987) (end 164.75 98.089998) (width 0.5) (layer F.Cu) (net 7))
 (segment (start 169.200011 90.865011) (end 169.200011 93.639987) (width 0.5) (layer F.Cu) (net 7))
 (segment (start 168.45 90.115) (end 169.200011 90.865011) (width 0.5) (layer F.Cu) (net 7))
 (segment (start 165.79 101.04) (end 166.75 101.04) (width 0.5) (layer F.Cu) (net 7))
 (segment (start 167.1 90.115) (end 168.45 90.115) (width 0.5) (layer F.Cu) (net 7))
 (segment (start 160.615 90.115) (end 167.1 90.115) (width 0.5) (layer F.Cu) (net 7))
 (segment (start 153.5 83) (end 160.615 90.115) (width 0.5) (layer F.Cu) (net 7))
 (segment (start 153.5 75.25) (end 153.5 83) (width 0.5) (layer F.Cu) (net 7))
 (segment (start 186.15 89.2) (end 188.55 89.2) (width 0.5) (layer F.Cu) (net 10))
 (segment (start 188.55 89.2) (end 191.25 86.5) (width 0.5) (layer F.Cu) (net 10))
 (segment (start 191.25 86.5) (end 191.25 82.25) (width 0.5) (layer F.Cu) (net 10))
 (segment (start 192 81.5) (end 194 81.5) (width 0.5) (layer F.Cu) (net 10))
 (segment (start 191.25 82.25) (end 192 81.5) (width 0.5) (layer F.Cu) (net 10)))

